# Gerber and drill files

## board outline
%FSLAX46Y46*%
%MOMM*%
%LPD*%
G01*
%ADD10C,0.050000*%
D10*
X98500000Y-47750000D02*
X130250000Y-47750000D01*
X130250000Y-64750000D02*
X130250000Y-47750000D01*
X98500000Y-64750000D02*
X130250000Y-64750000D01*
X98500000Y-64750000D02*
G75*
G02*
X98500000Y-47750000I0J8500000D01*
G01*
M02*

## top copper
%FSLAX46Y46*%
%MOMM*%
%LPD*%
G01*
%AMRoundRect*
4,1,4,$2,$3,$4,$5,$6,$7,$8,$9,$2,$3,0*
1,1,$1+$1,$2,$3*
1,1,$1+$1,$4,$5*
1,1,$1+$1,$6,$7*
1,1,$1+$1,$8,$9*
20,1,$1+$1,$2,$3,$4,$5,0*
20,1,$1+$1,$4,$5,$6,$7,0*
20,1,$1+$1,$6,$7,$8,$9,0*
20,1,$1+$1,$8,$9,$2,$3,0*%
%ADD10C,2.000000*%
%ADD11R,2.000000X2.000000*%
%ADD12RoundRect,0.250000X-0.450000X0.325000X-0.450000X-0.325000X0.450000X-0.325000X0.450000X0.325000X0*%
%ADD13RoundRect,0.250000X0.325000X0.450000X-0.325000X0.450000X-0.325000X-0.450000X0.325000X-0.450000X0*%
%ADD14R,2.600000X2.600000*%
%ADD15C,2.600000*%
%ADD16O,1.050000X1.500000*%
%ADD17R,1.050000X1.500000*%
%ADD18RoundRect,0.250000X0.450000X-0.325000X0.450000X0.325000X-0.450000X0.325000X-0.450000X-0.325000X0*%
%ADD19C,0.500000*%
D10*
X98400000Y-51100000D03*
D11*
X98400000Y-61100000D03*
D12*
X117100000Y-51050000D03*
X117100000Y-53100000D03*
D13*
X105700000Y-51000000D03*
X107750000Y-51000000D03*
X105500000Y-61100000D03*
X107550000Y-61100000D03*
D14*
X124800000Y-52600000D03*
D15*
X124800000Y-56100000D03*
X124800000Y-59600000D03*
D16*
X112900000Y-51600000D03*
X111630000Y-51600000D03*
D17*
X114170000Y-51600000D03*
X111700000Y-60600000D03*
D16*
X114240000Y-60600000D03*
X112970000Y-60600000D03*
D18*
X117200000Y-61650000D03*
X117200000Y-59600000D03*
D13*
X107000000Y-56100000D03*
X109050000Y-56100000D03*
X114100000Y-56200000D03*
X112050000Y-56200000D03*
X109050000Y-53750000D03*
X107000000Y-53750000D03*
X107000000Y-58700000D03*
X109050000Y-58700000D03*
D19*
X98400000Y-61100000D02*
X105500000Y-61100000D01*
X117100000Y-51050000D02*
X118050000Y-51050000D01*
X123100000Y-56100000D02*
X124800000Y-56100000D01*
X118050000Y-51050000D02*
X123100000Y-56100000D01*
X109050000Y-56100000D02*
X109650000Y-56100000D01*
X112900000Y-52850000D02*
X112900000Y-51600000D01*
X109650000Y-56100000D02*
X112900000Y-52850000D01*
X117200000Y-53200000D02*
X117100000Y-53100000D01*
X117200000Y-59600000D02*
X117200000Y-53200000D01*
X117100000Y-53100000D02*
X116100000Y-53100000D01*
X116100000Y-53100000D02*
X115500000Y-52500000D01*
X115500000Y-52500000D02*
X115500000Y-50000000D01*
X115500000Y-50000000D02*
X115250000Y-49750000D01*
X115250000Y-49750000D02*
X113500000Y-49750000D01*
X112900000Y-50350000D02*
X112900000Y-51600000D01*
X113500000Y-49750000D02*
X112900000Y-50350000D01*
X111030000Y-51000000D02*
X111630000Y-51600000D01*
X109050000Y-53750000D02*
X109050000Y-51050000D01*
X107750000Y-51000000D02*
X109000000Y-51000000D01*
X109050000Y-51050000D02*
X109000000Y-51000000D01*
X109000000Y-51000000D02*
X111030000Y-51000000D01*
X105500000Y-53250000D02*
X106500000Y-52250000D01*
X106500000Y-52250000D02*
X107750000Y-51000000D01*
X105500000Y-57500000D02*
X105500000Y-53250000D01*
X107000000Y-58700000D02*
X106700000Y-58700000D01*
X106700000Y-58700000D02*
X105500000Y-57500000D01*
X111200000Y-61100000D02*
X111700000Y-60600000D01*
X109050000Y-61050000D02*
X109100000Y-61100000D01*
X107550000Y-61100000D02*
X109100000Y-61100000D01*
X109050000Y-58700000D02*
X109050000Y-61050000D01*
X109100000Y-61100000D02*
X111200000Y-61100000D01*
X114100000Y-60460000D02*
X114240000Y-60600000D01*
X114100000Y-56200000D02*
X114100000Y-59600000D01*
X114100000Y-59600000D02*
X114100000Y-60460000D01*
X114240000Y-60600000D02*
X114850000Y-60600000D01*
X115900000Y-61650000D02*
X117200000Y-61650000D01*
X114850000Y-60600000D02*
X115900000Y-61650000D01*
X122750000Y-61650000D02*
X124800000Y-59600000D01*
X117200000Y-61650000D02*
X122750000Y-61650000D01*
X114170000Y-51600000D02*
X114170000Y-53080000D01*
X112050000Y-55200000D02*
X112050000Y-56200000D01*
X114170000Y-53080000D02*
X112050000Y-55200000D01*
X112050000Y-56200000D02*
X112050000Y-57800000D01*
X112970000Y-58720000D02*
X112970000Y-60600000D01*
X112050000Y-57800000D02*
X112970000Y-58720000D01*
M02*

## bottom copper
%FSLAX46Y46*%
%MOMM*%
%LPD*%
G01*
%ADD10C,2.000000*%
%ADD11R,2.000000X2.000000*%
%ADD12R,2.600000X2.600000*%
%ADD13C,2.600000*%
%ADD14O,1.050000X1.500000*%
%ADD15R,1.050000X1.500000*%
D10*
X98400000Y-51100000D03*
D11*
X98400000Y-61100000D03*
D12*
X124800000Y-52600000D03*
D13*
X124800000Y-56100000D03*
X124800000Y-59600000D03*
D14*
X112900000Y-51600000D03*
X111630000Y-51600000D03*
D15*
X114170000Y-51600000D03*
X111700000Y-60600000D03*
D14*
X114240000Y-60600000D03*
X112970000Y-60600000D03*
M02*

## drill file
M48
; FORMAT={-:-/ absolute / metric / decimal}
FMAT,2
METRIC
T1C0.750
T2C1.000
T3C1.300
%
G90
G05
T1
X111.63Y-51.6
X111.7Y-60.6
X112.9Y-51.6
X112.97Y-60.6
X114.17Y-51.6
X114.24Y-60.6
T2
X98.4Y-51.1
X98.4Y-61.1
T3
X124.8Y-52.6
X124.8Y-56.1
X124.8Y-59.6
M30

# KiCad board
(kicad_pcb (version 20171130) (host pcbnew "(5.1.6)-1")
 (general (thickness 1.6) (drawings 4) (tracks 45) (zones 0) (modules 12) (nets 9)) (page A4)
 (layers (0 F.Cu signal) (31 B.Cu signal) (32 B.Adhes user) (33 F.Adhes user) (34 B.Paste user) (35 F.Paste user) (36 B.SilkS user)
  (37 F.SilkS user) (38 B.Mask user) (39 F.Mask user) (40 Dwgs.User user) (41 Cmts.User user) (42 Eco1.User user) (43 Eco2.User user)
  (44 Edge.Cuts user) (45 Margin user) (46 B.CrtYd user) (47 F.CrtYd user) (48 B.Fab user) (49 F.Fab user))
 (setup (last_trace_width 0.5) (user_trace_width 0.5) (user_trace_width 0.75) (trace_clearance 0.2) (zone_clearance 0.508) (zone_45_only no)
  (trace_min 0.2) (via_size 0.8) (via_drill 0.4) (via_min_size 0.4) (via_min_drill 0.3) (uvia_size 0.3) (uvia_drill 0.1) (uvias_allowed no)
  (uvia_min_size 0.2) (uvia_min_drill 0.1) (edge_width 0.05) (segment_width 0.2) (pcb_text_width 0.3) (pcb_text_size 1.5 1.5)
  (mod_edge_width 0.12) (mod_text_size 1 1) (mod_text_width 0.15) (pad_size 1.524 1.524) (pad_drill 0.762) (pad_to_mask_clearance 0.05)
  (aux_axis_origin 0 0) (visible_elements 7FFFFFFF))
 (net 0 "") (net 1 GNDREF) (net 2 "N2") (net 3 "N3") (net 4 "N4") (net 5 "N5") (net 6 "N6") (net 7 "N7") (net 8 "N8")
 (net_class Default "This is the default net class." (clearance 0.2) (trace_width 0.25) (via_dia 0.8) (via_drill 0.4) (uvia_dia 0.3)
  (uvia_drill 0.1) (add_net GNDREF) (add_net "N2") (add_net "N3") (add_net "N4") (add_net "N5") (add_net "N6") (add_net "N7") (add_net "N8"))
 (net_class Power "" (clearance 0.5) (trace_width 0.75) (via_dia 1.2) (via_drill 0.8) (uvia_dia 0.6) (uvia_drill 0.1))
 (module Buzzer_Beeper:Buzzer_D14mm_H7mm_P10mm (layer F.Cu) (at 98.4 61.1 90)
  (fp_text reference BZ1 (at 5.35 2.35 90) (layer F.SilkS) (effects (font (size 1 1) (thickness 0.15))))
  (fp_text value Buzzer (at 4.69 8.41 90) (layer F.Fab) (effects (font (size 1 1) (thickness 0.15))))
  (pad 2 thru_hole circle (at 10 0 90) (size 2 2) (drill 1) (layers *.Cu *.Mask) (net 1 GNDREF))
  (pad 1 thru_hole rect (at 0 0 90) (size 2 2) (drill 1) (layers *.Cu *.Mask) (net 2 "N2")))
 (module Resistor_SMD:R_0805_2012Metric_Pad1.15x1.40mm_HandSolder (layer F.Cu) (at 117.1 52.075 270)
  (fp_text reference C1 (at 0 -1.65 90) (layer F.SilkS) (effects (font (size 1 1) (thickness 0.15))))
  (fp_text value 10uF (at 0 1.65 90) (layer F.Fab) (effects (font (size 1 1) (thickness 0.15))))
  (pad 1 smd roundrect (at -1.025 0 270) (size 1.15 1.4) (layers F.Cu F.Paste F.Mask) (roundrect_rratio 0.217391) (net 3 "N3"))
  (pad 2 smd roundrect (at 1.025 0 270) (size 1.15 1.4) (layers F.Cu F.Paste F.Mask) (roundrect_rratio 0.217391) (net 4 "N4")))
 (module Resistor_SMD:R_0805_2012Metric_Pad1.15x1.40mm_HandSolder (layer F.Cu) (at 106.725 51 180)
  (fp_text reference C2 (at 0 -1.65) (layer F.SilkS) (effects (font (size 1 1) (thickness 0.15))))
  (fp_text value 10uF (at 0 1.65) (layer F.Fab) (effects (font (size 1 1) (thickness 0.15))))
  (pad 2 smd roundrect (at 1.025 0 180) (size 1.15 1.4) (layers F.Cu F.Paste F.Mask) (roundrect_rratio 0.217391) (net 1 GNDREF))
  (pad 1 smd roundrect (at -1.025 0 180) (size 1.15 1.4) (layers F.Cu F.Paste F.Mask) (roundrect_rratio 0.217391) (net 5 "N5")))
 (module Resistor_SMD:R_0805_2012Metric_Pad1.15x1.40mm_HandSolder (layer F.Cu) (at 106.525 61.1 180)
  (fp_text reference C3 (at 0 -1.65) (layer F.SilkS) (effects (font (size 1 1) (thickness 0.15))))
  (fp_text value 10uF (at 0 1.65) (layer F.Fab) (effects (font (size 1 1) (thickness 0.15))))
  (pad 2 smd roundrect (at 1.025 0 180) (size 1.15 1.4) (layers F.Cu F.Paste F.Mask) (roundrect_rratio 0.217391) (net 2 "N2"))
  (pad 1 smd roundrect (at -1.025 0 180) (size 1.15 1.4) (layers F.Cu F.Paste F.Mask) (roundrect_rratio 0.217391) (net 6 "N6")))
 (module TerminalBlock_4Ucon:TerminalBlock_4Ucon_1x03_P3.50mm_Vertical (layer F.Cu) (at 124.8 52.6 270)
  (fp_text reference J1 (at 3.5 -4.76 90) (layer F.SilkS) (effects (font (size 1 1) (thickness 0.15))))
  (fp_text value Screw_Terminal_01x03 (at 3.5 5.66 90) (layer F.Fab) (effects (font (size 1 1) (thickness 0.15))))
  (pad 1 thru_hole rect (at 0 0 270) (size 2.6 2.6) (drill 1.3) (layers *.Cu *.Mask) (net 1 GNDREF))
  (pad 2 thru_hole circle (at 3.5 0 270) (size 2.6 2.6) (drill 1.3) (layers *.Cu *.Mask) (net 3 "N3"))
  (pad 3 thru_hole circle (at 7 0 270) (size 2.6 2.6) (drill 1.3) (layers *.Cu *.Mask) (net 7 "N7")))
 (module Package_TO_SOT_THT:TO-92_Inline (layer F.Cu) (at 114.17 51.6 180)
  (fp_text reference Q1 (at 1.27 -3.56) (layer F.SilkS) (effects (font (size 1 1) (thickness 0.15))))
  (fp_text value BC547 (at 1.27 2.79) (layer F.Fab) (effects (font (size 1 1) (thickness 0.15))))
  (pad 2 thru_hole oval (at 1.27 0 180) (size 1.05 1.5) (drill 0.75) (layers *.Cu *.Mask) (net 4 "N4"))
  (pad 3 thru_hole oval (at 2.54 0 180) (size 1.05 1.5) (drill 0.75) (layers *.Cu *.Mask) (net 5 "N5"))
  (pad 1 thru_hole rect (at 0 0 180) (size 1.05 1.5) (drill 0.75) (layers *.Cu *.Mask) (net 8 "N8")))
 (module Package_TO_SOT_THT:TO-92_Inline (layer F.Cu) (at 111.7 60.6)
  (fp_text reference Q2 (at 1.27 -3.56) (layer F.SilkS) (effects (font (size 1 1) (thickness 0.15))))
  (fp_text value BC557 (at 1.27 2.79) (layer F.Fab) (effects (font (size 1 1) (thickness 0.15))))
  (pad 1 thru_hole rect (at 0 0) (size 1.05 1.5) (drill 0.75) (layers *.Cu *.Mask) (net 6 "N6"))
  (pad 3 thru_hole oval (at 2.54 0) (size 1.05 1.5) (drill 0.75) (layers *.Cu *.Mask) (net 7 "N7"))
  (pad 2 thru_hole oval (at 1.27 0) (size 1.05 1.5) (drill 0.75) (layers *.Cu *.Mask) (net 8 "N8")))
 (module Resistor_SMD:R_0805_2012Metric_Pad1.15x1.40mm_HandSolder (layer F.Cu) (at 117.2 60.625 90)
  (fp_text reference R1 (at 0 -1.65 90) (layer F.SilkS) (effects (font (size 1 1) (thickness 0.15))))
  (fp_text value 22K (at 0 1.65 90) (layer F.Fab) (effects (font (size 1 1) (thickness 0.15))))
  (pad 1 smd roundrect (at -1.025 0 90) (size 1.15 1.4) (layers F.Cu F.Paste F.Mask) (roundrect_rratio 0.217391) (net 7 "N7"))
  (pad 2 smd roundrect (at 1.025 0 90) (size 1.15 1.4) (layers F.Cu F.Paste F.Mask) (roundrect_rratio 0.217391) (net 4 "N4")))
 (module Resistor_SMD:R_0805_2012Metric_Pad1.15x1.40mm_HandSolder (layer F.Cu) (at 108.025 56.1 180)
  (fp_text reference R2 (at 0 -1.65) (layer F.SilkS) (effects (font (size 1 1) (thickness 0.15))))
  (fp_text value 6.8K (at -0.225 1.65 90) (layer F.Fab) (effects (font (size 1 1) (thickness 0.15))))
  (pad 2 smd roundrect (at 1.025 0 180) (size 1.15 1.4) (layers F.Cu F.Paste F.Mask) (roundrect_rratio 0.217391) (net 1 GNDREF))
  (pad 1 smd roundrect (at -1.025 0 180) (size 1.15 1.4) (layers F.Cu F.Paste F.Mask) (roundrect_rratio 0.217391) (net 4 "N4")))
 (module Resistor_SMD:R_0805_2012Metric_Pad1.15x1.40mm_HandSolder (layer F.Cu) (at 113.075 56.2 180)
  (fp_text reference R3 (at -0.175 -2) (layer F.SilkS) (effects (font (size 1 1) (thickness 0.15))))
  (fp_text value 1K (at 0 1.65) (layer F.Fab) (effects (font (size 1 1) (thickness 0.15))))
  (pad 1 smd roundrect (at -1.025 0 180) (size 1.15 1.4) (layers F.Cu F.Paste F.Mask) (roundrect_rratio 0.217391) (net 7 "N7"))
  (pad 2 smd roundrect (at 1.025 0 180) (size 1.15 1.4) (layers F.Cu F.Paste F.Mask) (roundrect_rratio 0.217391) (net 8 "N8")))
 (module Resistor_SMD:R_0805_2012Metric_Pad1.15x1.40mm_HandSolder (layer F.Cu) (at 108.025 53.75 180)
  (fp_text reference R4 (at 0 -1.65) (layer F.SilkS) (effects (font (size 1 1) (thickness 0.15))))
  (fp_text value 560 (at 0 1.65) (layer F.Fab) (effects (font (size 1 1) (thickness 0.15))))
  (pad 1 smd roundrect (at -1.025 0 180) (size 1.15 1.4) (layers F.Cu F.Paste F.Mask) (roundrect_rratio 0.217391) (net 5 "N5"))
  (pad 2 smd roundrect (at 1.025 0 180) (size 1.15 1.4) (layers F.Cu F.Paste F.Mask) (roundrect_rratio 0.217391) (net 1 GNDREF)))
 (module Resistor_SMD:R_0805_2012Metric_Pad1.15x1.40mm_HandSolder (layer F.Cu) (at 108.025 58.7 180)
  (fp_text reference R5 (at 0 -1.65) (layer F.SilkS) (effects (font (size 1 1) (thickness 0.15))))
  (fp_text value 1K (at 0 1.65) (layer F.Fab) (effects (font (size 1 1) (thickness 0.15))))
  (pad 2 smd roundrect (at 1.025 0 180) (size 1.15 1.4) (layers F.Cu F.Paste F.Mask) (roundrect_rratio 0.217391) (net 5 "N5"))
  (pad 1 smd roundrect (at -1.025 0 180) (size 1.15 1.4) (layers F.Cu F.Paste F.Mask) (roundrect_rratio 0.217391) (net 6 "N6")))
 (gr_line (start 98.5 47.75) (end 130.25 47.75) (layer Edge.Cuts) (width 0.05))
 (gr_line (start 130.25 64.75) (end 130.25 47.75) (layer Edge.Cuts) (width 0.05))
 (gr_line (start 98.5 64.75) (end 130.25 64.75) (layer Edge.Cuts) (width 0.05))
 (gr_arc (start 98.5 56.25) (end 98.5 47.75) (angle -180) (layer Edge.Cuts) (width 0.05))
 (segment (start 98.4 61.1) (end 105.5 61.1) (width 0.5) (layer F.Cu) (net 2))
 (segment (start 117.1 51.05) (end 118.05 51.05) (width 0.5) (layer F.Cu) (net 3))
 (segment (start 123.1 56.1) (end 124.8 56.1) (width 0.5) (layer F.Cu) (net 3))
 (segment (start 118.05 51.05) (end 123.1 56.1) (width 0.5) (layer F.Cu) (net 3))
 (segment (start 109.05 56.1) (end 109.65 56.1) (width 0.5) (layer F.Cu) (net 4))
 (segment (start 112.9 52.85) (end 112.9 51.6) (width 0.5) (layer F.Cu) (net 4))
 (segment (start 109.65 56.1) (end 112.9 52.85) (width 0.5) (layer F.Cu) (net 4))
 (segment (start 117.2 53.2) (end 117.1 53.1) (width 0.5) (layer F.Cu) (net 4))
 (segment (start 117.2 59.6) (end 117.2 53.2) (width 0.5) (layer F.Cu) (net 4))
 (segment (start 117.1 53.1) (end 116.1 53.1) (width 0.5) (layer F.Cu) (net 4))
 (segment (start 116.1 53.1) (end 115.5 52.5) (width 0.5) (layer F.Cu) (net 4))
 (segment (start 115.5 52.5) (end 115.5 50) (width 0.5) (layer F.Cu) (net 4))
 (segment (start 115.5 50) (end 115.25 49.75) (width 0.5) (layer F.Cu) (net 4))
 (segment (start 115.25 49.75) (end 113.5 49.75) (width 0.5) (layer F.Cu) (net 4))
 (segment (start 112.9 50.35) (end 112.9 51.6) (width 0.5) (layer F.Cu) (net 4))
 (segment (start 113.5 49.75) (end 112.9 50.35) (width 0.5) (layer F.Cu) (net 4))
 (segment (start 111.03 51) (end 111.63 51.6) (width 0.5) (layer F.Cu) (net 5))
 (segment (start 109.05 53.75) (end 109.05 51.05) (width 0.5) (layer F.Cu) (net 5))
 (segment (start 107.75 51) (end 109 51) (width 0.5) (layer F.Cu) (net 5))
 (segment (start 109.05 51.05) (end 109 51) (width 0.5) (layer F.Cu) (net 5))
 (segment (start 109 51) (end 111.03 51) (width 0.5) (layer F.Cu) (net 5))
 (segment (start 105.5 53.25) (end 106.5 52.25) (width 0.5) (layer F.Cu) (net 5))
 (segment (start 106.5 52.25) (end 107.75 51) (width 0.5) (layer F.Cu) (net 5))
 (segment (start 105.5 57.5) (end 105.5 53.25) (width 0.5) (layer F.Cu) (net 5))
 (segment (start 107 58.7) (end 106.7 58.7) (width 0.5) (layer F.Cu) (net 5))
 (segment (start 106.7 58.7) (end 105.5 57.5) (width 0.5) (layer F.Cu) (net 5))
 (segment (start 111.2 61.1) (end 111.7 60.6) (width 0.5) (layer F.Cu) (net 6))
 (segment (start 109.05 61.05) (end 109.1 61.1) (width 0.5) (layer F.Cu) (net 6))
 (segment (start 107.55 61.1) (end 109.1 61.1) (width 0.5) (layer F.Cu) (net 6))
 (segment (start 109.05 58.7) (end 109.05 61.05) (width 0.5) (layer F.Cu) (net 6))
 (segment (start 109.1 61.1) (end 111.2 61.1) (width 0.5) (layer F.Cu) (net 6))
 (segment (start 114.1 60.46) (end 114.24 60.6) (width 0.5) (layer F.Cu) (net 7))
 (segment (start 114.1 56.2) (end 114.1 59.6) (width 0.5) (layer F.Cu) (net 7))
 (segment (start 114.1 59.6) (end 114.1 60.46) (width 0.5) (layer F.Cu) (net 7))
 (segment (start 114.24 60.6) (end 114.85 60.6) (width 0.5) (layer F.Cu) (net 7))
 (segment (start 115.9 61.65) (end 117.2 61.65) (width 0.5) (layer F.Cu) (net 7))
 (segment (start 114.85 60.6) (end 115.9 61.65) (width 0.5) (layer F.Cu) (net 7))
 (segment (start 122.75 61.65) (end 124.8 59.6) (width 0.5) (layer F.Cu) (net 7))
 (segment (start 117.2 61.65) (end 122.75 61.65) (width 0.5) (layer F.Cu) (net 7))
 (segment (start 114.17 51.6) (end 114.17 53.08) (width 0.5) (layer F.Cu) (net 8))
 (segment (start 112.05 55.2) (end 112.05 56.2) (width 0.5) (layer F.Cu) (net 8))
 (segment (start 114.17 53.08) (end 112.05 55.2) (width 0.5) (layer F.Cu) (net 8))
 (segment (start 112.05 56.2) (end 112.05 57.8) (width 0.5) (layer F.Cu) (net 8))
 (segment (start 112.97 58.72) (end 112.97 60.6) (width 0.5) (layer F.Cu) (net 8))
 (segment (start 112.05 57.8) (end 112.97 58.72) (width 0.5) (layer F.Cu) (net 8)))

